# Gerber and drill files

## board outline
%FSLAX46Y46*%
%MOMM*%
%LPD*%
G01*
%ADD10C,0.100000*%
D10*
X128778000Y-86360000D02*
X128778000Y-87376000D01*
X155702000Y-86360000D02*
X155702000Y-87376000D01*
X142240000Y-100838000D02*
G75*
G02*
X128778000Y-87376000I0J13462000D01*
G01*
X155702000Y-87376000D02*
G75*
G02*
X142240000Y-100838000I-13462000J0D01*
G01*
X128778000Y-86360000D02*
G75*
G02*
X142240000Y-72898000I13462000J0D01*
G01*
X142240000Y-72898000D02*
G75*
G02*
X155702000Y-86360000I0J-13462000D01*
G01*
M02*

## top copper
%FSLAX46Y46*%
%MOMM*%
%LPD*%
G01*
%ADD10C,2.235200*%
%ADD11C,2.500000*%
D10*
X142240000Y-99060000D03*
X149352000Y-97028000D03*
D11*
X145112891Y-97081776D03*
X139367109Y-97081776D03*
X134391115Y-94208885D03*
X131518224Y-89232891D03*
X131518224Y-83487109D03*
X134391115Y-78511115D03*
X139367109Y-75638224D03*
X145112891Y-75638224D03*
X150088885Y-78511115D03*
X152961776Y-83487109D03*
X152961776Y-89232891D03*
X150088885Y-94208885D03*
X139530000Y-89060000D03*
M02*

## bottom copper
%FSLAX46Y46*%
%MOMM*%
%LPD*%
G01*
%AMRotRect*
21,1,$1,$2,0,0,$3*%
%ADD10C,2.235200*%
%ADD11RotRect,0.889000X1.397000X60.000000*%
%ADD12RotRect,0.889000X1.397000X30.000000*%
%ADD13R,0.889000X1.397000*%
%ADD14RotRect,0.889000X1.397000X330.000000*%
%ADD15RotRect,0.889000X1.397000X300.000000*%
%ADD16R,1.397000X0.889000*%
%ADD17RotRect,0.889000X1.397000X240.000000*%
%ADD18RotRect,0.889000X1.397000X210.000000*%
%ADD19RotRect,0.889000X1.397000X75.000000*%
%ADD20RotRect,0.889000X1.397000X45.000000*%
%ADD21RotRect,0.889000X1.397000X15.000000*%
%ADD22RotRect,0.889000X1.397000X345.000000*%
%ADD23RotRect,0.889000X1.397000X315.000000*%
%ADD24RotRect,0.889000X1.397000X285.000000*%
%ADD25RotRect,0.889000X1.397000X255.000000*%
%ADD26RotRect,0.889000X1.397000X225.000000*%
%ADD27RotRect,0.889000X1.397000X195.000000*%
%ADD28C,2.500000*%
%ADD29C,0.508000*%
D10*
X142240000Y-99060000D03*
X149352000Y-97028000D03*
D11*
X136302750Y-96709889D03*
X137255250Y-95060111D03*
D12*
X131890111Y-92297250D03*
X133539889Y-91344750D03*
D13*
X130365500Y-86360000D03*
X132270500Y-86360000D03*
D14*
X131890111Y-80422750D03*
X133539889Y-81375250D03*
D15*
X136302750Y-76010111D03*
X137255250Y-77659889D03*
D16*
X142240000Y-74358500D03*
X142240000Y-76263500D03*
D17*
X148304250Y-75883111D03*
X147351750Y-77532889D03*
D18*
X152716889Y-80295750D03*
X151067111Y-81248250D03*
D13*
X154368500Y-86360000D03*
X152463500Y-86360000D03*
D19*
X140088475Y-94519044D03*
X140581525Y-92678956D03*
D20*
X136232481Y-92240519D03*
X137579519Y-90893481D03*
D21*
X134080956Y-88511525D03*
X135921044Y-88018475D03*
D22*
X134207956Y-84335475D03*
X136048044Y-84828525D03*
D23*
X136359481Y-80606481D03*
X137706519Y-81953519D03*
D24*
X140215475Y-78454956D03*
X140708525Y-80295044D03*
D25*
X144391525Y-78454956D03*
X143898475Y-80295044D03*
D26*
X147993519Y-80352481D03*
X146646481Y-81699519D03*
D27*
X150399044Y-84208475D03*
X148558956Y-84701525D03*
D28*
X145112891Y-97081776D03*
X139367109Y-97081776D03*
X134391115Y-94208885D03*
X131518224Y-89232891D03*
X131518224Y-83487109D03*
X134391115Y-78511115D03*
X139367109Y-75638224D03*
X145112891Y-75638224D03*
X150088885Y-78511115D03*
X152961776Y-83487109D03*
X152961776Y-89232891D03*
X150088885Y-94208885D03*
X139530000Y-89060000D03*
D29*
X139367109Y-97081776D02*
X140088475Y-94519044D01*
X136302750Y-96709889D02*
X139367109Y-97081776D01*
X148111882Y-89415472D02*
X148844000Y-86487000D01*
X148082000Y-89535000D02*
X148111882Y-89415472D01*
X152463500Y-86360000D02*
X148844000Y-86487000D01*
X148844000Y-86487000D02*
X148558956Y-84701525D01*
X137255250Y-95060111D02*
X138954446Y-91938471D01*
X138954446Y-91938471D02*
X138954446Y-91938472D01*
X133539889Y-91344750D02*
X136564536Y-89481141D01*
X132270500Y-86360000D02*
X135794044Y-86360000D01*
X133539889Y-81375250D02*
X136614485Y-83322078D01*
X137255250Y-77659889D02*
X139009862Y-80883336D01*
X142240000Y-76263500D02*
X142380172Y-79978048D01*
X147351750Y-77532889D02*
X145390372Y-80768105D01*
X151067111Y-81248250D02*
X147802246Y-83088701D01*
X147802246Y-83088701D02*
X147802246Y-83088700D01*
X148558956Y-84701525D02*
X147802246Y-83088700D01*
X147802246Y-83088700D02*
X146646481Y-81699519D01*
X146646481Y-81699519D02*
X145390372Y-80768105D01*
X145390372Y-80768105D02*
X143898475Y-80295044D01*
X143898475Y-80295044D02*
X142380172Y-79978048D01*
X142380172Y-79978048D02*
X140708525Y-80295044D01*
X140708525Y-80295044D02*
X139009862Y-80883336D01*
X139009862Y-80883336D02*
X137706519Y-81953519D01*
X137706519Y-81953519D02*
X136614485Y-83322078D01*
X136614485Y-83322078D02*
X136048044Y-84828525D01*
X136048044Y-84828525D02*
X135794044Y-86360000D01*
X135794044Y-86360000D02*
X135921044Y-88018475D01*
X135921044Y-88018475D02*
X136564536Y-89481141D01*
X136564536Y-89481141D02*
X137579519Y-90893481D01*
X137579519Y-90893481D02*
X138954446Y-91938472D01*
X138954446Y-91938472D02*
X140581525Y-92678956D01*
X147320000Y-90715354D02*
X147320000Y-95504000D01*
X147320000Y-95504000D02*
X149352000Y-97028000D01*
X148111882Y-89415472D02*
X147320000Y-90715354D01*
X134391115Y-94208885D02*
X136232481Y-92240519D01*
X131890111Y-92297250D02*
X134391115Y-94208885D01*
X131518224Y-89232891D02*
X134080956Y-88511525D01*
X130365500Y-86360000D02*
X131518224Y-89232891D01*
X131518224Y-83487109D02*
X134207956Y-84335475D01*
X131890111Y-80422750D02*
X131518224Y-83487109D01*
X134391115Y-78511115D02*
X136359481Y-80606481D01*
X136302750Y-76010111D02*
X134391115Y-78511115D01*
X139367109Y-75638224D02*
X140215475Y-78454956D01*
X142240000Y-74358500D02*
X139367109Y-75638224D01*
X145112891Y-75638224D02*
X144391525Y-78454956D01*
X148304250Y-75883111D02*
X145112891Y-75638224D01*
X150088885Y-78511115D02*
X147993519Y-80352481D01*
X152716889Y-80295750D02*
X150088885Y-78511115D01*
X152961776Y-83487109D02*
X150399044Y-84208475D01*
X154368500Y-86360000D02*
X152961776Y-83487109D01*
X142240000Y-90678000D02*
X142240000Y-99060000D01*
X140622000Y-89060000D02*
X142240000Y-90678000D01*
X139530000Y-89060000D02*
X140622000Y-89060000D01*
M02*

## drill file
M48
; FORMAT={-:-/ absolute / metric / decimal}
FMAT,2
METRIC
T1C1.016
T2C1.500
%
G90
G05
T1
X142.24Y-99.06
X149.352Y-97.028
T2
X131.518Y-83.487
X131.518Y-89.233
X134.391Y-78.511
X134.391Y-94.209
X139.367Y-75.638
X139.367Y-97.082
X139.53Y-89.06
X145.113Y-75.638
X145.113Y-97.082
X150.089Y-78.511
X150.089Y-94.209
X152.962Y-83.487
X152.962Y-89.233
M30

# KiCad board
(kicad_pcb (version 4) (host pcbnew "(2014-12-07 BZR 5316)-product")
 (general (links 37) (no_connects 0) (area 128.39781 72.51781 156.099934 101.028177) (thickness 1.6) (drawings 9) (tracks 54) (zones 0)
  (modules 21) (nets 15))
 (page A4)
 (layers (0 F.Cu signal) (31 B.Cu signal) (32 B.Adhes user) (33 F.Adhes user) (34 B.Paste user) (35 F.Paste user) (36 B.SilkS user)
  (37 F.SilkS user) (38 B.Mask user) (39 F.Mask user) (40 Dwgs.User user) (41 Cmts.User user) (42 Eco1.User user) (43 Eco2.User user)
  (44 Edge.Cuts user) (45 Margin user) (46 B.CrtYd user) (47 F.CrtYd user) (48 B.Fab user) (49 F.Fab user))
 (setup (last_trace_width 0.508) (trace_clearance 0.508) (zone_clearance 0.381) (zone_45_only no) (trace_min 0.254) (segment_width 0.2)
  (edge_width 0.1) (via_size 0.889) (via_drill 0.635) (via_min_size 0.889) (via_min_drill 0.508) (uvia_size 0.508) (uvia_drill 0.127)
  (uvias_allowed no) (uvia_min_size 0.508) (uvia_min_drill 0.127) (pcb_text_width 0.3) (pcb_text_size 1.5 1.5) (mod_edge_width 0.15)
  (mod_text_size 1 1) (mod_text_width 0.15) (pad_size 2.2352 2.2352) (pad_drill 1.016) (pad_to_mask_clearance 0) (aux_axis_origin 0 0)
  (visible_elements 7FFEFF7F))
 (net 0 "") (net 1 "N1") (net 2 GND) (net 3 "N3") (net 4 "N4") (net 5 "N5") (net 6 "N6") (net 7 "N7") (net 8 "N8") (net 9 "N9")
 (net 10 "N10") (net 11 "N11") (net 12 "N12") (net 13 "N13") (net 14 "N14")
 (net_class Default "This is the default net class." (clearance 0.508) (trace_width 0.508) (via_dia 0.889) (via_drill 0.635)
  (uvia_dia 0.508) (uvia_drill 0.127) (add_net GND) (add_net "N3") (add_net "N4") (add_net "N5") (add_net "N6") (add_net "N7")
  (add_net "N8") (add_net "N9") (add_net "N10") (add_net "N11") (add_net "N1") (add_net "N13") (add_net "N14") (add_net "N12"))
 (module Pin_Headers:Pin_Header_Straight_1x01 (layer F.Cu) (at 142.24 99.06 90)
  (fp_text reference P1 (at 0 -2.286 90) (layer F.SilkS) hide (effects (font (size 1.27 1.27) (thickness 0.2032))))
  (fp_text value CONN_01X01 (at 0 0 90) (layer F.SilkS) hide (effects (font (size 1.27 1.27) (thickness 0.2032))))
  (pad 1 thru_hole circle (at 0 0 90) (size 2.2352 2.2352) (drill 1.016) (layers *.Cu *.Mask F.SilkS) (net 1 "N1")))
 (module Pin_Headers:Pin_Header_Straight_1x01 (layer F.Cu) (at 149.352 97.028 30)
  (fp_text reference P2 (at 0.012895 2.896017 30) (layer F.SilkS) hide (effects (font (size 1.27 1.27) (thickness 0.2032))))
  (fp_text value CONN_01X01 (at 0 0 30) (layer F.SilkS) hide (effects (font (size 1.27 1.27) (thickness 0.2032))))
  (pad 1 thru_hole circle (at 0 0 30) (size 2.2352 2.2352) (drill 1.016) (layers *.Cu *.Mask F.SilkS) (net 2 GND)))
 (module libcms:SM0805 (layer B.Cu) (at 136.779 95.885 60)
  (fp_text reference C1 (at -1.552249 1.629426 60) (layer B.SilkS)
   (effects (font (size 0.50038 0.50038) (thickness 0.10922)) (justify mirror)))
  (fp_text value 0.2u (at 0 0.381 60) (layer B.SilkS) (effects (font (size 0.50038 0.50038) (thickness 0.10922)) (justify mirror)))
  (pad 1 smd rect (at -0.9525 0 60) (size 0.889 1.397) (layers B.Cu B.Paste B.Mask) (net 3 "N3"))
  (pad 2 smd rect (at 0.9525 0 60) (size 0.889 1.397) (layers B.Cu B.Paste B.Mask) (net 2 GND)))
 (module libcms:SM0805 (layer B.Cu) (at 132.715 91.821 30)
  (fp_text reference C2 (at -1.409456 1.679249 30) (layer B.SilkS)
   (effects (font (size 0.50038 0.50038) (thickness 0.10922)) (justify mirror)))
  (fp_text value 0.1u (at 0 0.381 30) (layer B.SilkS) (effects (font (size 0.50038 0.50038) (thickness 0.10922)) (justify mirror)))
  (pad 1 smd rect (at -0.9525 0 30) (size 0.889 1.397) (layers B.Cu B.Paste B.Mask) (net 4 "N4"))
  (pad 2 smd rect (at 0.9525 0 30) (size 0.889 1.397) (layers B.Cu B.Paste B.Mask) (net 2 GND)))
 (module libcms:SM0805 (layer B.Cu) (at 131.318 86.36)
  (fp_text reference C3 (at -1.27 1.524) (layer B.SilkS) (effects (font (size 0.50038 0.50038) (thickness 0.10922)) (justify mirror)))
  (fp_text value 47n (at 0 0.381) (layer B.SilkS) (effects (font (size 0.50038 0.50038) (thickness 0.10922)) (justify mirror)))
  (pad 1 smd rect (at -0.9525 0) (size 0.889 1.397) (layers B.Cu B.Paste B.Mask) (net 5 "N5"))
  (pad 2 smd rect (at 0.9525 0) (size 0.889 1.397) (layers B.Cu B.Paste B.Mask) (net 2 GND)))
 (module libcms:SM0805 (layer B.Cu) (at 132.715 80.899 330)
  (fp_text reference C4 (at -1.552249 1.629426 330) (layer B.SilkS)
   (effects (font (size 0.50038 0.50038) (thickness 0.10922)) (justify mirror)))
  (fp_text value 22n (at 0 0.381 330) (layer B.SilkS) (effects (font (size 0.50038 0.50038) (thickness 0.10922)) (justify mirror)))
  (pad 1 smd rect (at -0.9525 0 330) (size 0.889 1.397) (layers B.Cu B.Paste B.Mask) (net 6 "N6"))
  (pad 2 smd rect (at 0.9525 0 330) (size 0.889 1.397) (layers B.Cu B.Paste B.Mask) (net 2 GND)))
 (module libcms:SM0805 (layer B.Cu) (at 136.779 76.835 300)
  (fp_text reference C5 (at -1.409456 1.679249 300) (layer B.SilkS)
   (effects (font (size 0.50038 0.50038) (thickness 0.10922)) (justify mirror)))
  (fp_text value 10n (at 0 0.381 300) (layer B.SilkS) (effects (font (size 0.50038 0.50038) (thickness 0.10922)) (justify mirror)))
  (pad 1 smd rect (at -0.9525 0 300) (size 0.889 1.397) (layers B.Cu B.Paste B.Mask) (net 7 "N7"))
  (pad 2 smd rect (at 0.9525 0 300) (size 0.889 1.397) (layers B.Cu B.Paste B.Mask) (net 2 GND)))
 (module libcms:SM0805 (layer B.Cu) (at 142.24 75.311 270)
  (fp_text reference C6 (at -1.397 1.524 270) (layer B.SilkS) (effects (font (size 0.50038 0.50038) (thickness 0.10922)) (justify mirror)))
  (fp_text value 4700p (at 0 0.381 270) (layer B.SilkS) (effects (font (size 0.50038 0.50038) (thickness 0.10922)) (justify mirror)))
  (pad 1 smd rect (at -0.9525 0 270) (size 0.889 1.397) (layers B.Cu B.Paste B.Mask) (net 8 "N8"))
  (pad 2 smd rect (at 0.9525 0 270) (size 0.889 1.397) (layers B.Cu B.Paste B.Mask) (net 2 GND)))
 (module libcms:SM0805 (layer B.Cu) (at 147.828 76.708 240)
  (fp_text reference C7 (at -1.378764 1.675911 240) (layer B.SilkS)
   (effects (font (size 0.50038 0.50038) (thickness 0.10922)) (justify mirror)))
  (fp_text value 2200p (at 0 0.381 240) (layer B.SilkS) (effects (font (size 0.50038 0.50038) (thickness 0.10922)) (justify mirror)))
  (pad 1 smd rect (at -0.9525 0 240) (size 0.889 1.397) (layers B.Cu B.Paste B.Mask) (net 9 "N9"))
  (pad 2 smd rect (at 0.9525 0 240) (size 0.889 1.397) (layers B.Cu B.Paste B.Mask) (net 2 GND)))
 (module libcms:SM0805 (layer B.Cu) (at 151.892 80.772 210)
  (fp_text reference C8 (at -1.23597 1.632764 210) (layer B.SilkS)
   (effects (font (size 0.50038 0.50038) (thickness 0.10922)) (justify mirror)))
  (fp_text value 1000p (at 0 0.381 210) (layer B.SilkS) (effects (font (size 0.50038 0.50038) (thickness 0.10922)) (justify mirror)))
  (pad 1 smd rect (at -0.9525 0 210) (size 0.889 1.397) (layers B.Cu B.Paste B.Mask) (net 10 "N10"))
  (pad 2 smd rect (at 0.9525 0 210) (size 0.889 1.397) (layers B.Cu B.Paste B.Mask) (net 2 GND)))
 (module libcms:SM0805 (layer B.Cu) (at 153.416 86.36 180)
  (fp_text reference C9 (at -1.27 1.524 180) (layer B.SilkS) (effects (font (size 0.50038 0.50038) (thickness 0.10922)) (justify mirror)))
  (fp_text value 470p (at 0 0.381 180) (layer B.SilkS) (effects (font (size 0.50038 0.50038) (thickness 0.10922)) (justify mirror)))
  (pad 1 smd rect (at -0.9525 0 180) (size 0.889 1.397) (layers B.Cu B.Paste B.Mask) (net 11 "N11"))
  (pad 2 smd rect (at 0.9525 0 180) (size 0.889 1.397) (layers B.Cu B.Paste B.Mask) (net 2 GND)))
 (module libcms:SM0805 (layer B.Cu) (at 140.335 93.599 75)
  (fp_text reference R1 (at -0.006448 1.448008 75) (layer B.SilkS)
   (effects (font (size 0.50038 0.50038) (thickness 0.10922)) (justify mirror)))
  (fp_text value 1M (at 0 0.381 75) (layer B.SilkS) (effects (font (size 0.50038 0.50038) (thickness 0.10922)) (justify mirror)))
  (pad 1 smd rect (at -0.9525 0 75) (size 0.889 1.397) (layers B.Cu B.Paste B.Mask) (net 3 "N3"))
  (pad 2 smd rect (at 0.9525 0 75) (size 0.889 1.397) (layers B.Cu B.Paste B.Mask) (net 2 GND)))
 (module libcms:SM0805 (layer B.Cu) (at 136.906 91.567 45)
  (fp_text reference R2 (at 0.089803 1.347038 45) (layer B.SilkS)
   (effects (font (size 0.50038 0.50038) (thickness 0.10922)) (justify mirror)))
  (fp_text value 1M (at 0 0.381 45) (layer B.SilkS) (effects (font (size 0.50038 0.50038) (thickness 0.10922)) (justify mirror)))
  (pad 1 smd rect (at -0.9525 0 45) (size 0.889 1.397) (layers B.Cu B.Paste B.Mask) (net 4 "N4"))
  (pad 2 smd rect (at 0.9525 0 45) (size 0.889 1.397) (layers B.Cu B.Paste B.Mask) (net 2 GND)))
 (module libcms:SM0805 (layer B.Cu) (at 135.001 88.265 15)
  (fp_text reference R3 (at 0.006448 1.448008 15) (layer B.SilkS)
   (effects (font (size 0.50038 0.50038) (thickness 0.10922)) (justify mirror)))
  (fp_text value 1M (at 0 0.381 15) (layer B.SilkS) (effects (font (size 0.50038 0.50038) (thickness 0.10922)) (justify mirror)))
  (pad 1 smd rect (at -0.9525 0 15) (size 0.889 1.397) (layers B.Cu B.Paste B.Mask) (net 5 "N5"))
  (pad 2 smd rect (at 0.9525 0 15) (size 0.889 1.397) (layers B.Cu B.Paste B.Mask) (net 2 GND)))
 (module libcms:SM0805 (layer B.Cu) (at 135.128 84.582 345)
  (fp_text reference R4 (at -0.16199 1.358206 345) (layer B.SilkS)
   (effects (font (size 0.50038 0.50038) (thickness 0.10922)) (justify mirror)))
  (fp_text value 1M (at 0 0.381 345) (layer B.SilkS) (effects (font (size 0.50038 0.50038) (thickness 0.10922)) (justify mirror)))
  (pad 1 smd rect (at -0.9525 0 345) (size 0.889 1.397) (layers B.Cu B.Paste B.Mask) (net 6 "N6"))
  (pad 2 smd rect (at 0.9525 0 345) (size 0.889 1.397) (layers B.Cu B.Paste B.Mask) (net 2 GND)))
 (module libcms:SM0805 (layer B.Cu) (at 137.033 81.28 315)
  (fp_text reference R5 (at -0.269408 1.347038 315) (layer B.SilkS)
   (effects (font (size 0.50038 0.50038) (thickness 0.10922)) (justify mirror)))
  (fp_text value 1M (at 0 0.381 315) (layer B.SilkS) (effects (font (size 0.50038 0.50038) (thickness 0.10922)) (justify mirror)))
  (pad 1 smd rect (at -0.9525 0 315) (size 0.889 1.397) (layers B.Cu B.Paste B.Mask) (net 7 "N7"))
  (pad 2 smd rect (at 0.9525 0 315) (size 0.889 1.397) (layers B.Cu B.Paste B.Mask) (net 2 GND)))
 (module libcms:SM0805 (layer B.Cu) (at 140.462 79.375 285)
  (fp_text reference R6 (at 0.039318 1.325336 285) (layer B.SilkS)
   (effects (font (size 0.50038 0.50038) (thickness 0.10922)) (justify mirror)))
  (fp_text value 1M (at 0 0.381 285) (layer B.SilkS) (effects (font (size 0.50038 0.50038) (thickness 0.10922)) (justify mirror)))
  (pad 1 smd rect (at -0.9525 0 285) (size 0.889 1.397) (layers B.Cu B.Paste B.Mask) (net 8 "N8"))
  (pad 2 smd rect (at 0.9525 0 285) (size 0.889 1.397) (layers B.Cu B.Paste B.Mask) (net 2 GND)))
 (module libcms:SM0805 (layer B.Cu) (at 144.145 79.375 255)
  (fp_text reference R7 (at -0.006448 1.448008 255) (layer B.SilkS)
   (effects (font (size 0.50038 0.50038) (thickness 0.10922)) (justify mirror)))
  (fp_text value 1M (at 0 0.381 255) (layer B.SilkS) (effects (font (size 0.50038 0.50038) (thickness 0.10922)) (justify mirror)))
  (pad 1 smd rect (at -0.9525 0 255) (size 0.889 1.397) (layers B.Cu B.Paste B.Mask) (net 9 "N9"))
  (pad 2 smd rect (at 0.9525 0 255) (size 0.889 1.397) (layers B.Cu B.Paste B.Mask) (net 2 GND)))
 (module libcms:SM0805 (layer B.Cu) (at 147.32 81.026 225)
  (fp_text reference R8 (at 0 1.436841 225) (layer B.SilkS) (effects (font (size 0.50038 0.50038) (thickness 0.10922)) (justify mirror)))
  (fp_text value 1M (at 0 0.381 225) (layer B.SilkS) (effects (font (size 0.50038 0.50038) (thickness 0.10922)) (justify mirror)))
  (pad 1 smd rect (at -0.9525 0 225) (size 0.889 1.397) (layers B.Cu B.Paste B.Mask) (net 10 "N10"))
  (pad 2 smd rect (at 0.9525 0 225) (size 0.889 1.397) (layers B.Cu B.Paste B.Mask) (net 2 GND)))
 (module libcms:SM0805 (layer B.Cu) (at 149.479 84.455 195)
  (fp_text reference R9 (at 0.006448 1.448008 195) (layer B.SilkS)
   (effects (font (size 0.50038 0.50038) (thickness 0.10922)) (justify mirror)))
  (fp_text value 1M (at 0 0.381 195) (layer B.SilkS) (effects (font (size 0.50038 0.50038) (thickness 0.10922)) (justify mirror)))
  (pad 1 smd rect (at -0.9525 0 195) (size 0.889 1.397) (layers B.Cu B.Paste B.Mask) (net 11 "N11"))
  (pad 2 smd rect (at 0.9525 0 195) (size 0.889 1.397) (layers B.Cu B.Paste B.Mask) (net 2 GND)))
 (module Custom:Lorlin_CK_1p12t (layer F.Cu) (at 142.24 86.36)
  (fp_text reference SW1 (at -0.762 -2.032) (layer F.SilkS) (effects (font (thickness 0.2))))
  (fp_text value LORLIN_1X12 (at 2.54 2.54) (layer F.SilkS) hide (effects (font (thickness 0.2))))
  (pad 12 thru_hole circle (at 2.872891 10.721776) (size 2.5 2.5) (drill 1.5) (layers *.Cu *.Mask F.SilkS) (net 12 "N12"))
  (pad 1 thru_hole circle (at -2.872891 10.721776) (size 2.5 2.5) (drill 1.5) (layers *.Cu *.Mask F.SilkS) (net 3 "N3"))
  (pad 2 thru_hole circle (at -7.848885 7.848885) (size 2.5 2.5) (drill 1.5) (layers *.Cu *.Mask F.SilkS) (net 4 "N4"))
  (pad 3 thru_hole circle (at -10.721776 2.872891) (size 2.5 2.5) (drill 1.5) (layers *.Cu *.Mask F.SilkS) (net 5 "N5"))
  (pad 4 thru_hole circle (at -10.721776 -2.872891) (size 2.5 2.5) (drill 1.5) (layers *.Cu *.Mask F.SilkS) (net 6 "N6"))
  (pad 5 thru_hole circle (at -7.848885 -7.848885) (size 2.5 2.5) (drill 1.5) (layers *.Cu *.Mask F.SilkS) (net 7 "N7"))
  (pad 6 thru_hole circle (at -2.872891 -10.721776) (size 2.5 2.5) (drill 1.5) (layers *.Cu *.Mask F.SilkS) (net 8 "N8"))
  (pad 7 thru_hole circle (at 2.872891 -10.721776) (size 2.5 2.5) (drill 1.5) (layers *.Cu *.Mask F.SilkS) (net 9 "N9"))
  (pad 8 thru_hole circle (at 7.848885 -7.848885) (size 2.5 2.5) (drill 1.5) (layers *.Cu *.Mask F.SilkS) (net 10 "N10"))
  (pad 9 thru_hole circle (at 10.721776 -2.872891) (size 2.5 2.5) (drill 1.5) (layers *.Cu *.Mask F.SilkS) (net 11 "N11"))
  (pad 10 thru_hole circle (at 10.721776 2.872891) (size 2.5 2.5) (drill 1.5) (layers *.Cu *.Mask F.SilkS) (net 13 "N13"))
  (pad 11 thru_hole circle (at 7.848885 7.848885) (size 2.5 2.5) (drill 1.5) (layers *.Cu *.Mask F.SilkS) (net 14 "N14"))
  (pad A thru_hole circle (at -2.71 2.7) (size 2.5 2.5) (drill 1.5) (layers *.Cu *.Mask F.SilkS) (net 1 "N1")))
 (gr_line (start 128.778 86.36) (end 128.778 87.376) (angle 90) (layer Edge.Cuts) (width 0.1))
 (gr_line (start 155.702 86.36) (end 155.702 87.376) (angle 90) (layer Edge.Cuts) (width 0.1))
 (gr_arc (start 142.24 87.376) (end 142.24 100.838) (angle 90) (layer Edge.Cuts) (width 0.1))
 (gr_arc (start 142.24 87.376) (end 155.702 87.376) (angle 90) (layer Edge.Cuts) (width 0.1))
 (gr_arc (start 142.24 86.36) (end 128.778 86.36) (angle 90) (layer Edge.Cuts) (width 0.1))
 (gr_arc (start 142.24 86.36) (end 142.24 72.898) (angle 90) (layer Edge.Cuts) (width 0.1))
 (segment (start 139.367109 97.081776) (end 140.088475 94.519044) (width 0.508) (layer B.Cu) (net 3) (status 10))
 (segment (start 136.30275 96.709889) (end 139.367109 97.081776) (width 0.508) (layer B.Cu) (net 3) (status 20))
 (segment (start 148.111882 89.415472) (end 148.844 86.487) (width 0.508) (layer B.Cu) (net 2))
 (segment (start 148.082 89.535) (end 148.111882 89.415472) (width 0.508) (layer B.Cu) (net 2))
 (segment (start 152.4635 86.36) (end 148.844 86.487) (width 0.508) (layer B.Cu) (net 2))
 (segment (start 148.844 86.487) (end 148.558956 84.701525) (width 0.508) (layer B.Cu) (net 2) (status 20))
 (segment (start 137.25525 95.060111) (end 138.954446 91.938471) (width 0.508) (layer B.Cu) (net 2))
 (segment (start 138.954446 91.938471) (end 138.954446 91.938472) (width 0.508) (layer B.Cu) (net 2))
 (segment (start 133.539889 91.34475) (end 136.564536 89.481141) (width 0.508) (layer B.Cu) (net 2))
 (segment (start 132.2705 86.36) (end 135.794044 86.36) (width 0.508) (layer B.Cu) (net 2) (status 10))
 (segment (start 133.539889 81.37525) (end 136.614485 83.322078) (width 0.508) (layer B.Cu) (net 2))
 (segment (start 137.25525 77.659889) (end 139.009862 80.883336) (width 0.508) (layer B.Cu) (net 2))
 (segment (start 142.24 76.2635) (end 142.380172 79.978048) (width 0.508) (layer B.Cu) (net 2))
 (segment (start 147.35175 77.532889) (end 145.390372 80.768105) (width 0.508) (layer B.Cu) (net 2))
 (segment (start 151.067111 81.24825) (end 147.802246 83.088701) (width 0.508) (layer B.Cu) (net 2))
 (segment (start 147.802246 83.088701) (end 147.802246 83.0887) (width 0.508) (layer B.Cu) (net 2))
 (segment (start 148.558956 84.701525) (end 147.802246 83.0887) (width 0.508) (layer B.Cu) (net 2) (status 10))
 (segment (start 147.802246 83.0887) (end 146.646481 81.699519) (width 0.508) (layer B.Cu) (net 2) (status 20))
 (segment (start 146.646481 81.699519) (end 145.390372 80.768105) (width 0.508) (layer B.Cu) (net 2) (status 10))
 (segment (start 145.390372 80.768105) (end 143.898475 80.295044) (width 0.508) (layer B.Cu) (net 2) (status 20))
 (segment (start 143.898475 80.295044) (end 142.380172 79.978048) (width 0.508) (layer B.Cu) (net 2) (status 10))
 (segment (start 142.380172 79.978048) (end 140.708525 80.295044) (width 0.508) (layer B.Cu) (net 2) (status 20))
 (segment (start 140.708525 80.295044) (end 139.009862 80.883336) (width 0.508) (layer B.Cu) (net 2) (status 10))
 (segment (start 139.009862 80.883336) (end 137.706519 81.953519) (width 0.508) (layer B.Cu) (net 2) (status 20))
 (segment (start 137.706519 81.953519) (end 136.614485 83.322078) (width 0.508) (layer B.Cu) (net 2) (status 10))
 (segment (start 136.614485 83.322078) (end 136.048044 84.828525) (width 0.508) (layer B.Cu) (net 2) (status 20))
 (segment (start 136.048044 84.828525) (end 135.794044 86.36) (width 0.508) (layer B.Cu) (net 2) (status 10))
 (segment (start 135.794044 86.36) (end 135.921044 88.018475) (width 0.508) (layer B.Cu) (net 2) (status 20))
 (segment (start 135.921044 88.018475) (end 136.564536 89.481141) (width 0.508) (layer B.Cu) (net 2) (status 10))
 (segment (start 136.564536 89.481141) (end 137.579519 90.893481) (width 0.508) (layer B.Cu) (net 2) (status 20))
 (segment (start 137.579519 90.893481) (end 138.954446 91.938472) (width 0.508) (layer B.Cu) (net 2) (status 10))
 (segment (start 138.954446 91.938472) (end 140.581525 92.678956) (width 0.508) (layer B.Cu) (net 2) (status 20))
 (segment (start 147.32 90.715354) (end 147.32 95.504) (width 0.508) (layer B.Cu) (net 2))
 (segment (start 147.32 95.504) (end 149.352 97.028) (width 0.508) (layer B.Cu) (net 2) (status 20))
 (segment (start 148.111882 89.415472) (end 147.32 90.715354) (width 0.508) (layer B.Cu) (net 2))
 (segment (start 134.391115 94.208885) (end 136.232481 92.240519) (width 0.508) (layer B.Cu) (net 4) (status 10))
 (segment (start 131.890111 92.29725) (end 134.391115 94.208885) (width 0.508) (layer B.Cu) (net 4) (status 20))
 (segment (start 131.518224 89.232891) (end 134.080956 88.511525) (width 0.508) (layer B.Cu) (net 5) (status 10))
 (segment (start 130.3655 86.36) (end 131.518224 89.232891) (width 0.508) (layer B.Cu) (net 5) (status 20))
 (segment (start 131.518224 83.487109) (end 134.207956 84.335475) (width 0.508) (layer B.Cu) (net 6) (status 10))
 (segment (start 131.890111 80.42275) (end 131.518224 83.487109) (width 0.508) (layer B.Cu) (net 6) (status 20))
 (segment (start 134.391115 78.511115) (end 136.359481 80.606481) (width 0.508) (layer B.Cu) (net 7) (status 10))
 (segment (start 136.30275 76.010111) (end 134.391115 78.511115) (width 0.508) (layer B.Cu) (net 7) (status 20))
 (segment (start 139.367109 75.638224) (end 140.215475 78.454956) (width 0.508) (layer B.Cu) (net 8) (status 10))
 (segment (start 142.24 74.3585) (end 139.367109 75.638224) (width 0.508) (layer B.Cu) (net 8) (status 20))
 (segment (start 145.112891 75.638224) (end 144.391525 78.454956) (width 0.508) (layer B.Cu) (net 9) (status 10))
 (segment (start 148.30425 75.883111) (end 145.112891 75.638224) (width 0.508) (layer B.Cu) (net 9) (status 20))
 (segment (start 150.088885 78.511115) (end 147.993519 80.352481) (width 0.508) (layer B.Cu) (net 10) (status 10))
 (segment (start 152.716889 80.29575) (end 150.088885 78.511115) (width 0.508) (layer B.Cu) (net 10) (status 20))
 (segment (start 152.961776 83.487109) (end 150.399044 84.208475) (width 0.508) (layer B.Cu) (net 11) (status 10))
 (segment (start 154.3685 86.36) (end 152.961776 83.487109) (width 0.508) (layer B.Cu) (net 11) (status 20))
 (segment (start 142.24 90.678) (end 142.24 99.06) (width 0.508) (layer B.Cu) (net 1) (status 20))
 (segment (start 140.622 89.06) (end 142.24 90.678) (width 0.508) (layer B.Cu) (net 1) (status 10))
 (segment (start 139.53 89.06) (end 140.622 89.06) (width 0.508) (layer B.Cu) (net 1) (status 30)))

